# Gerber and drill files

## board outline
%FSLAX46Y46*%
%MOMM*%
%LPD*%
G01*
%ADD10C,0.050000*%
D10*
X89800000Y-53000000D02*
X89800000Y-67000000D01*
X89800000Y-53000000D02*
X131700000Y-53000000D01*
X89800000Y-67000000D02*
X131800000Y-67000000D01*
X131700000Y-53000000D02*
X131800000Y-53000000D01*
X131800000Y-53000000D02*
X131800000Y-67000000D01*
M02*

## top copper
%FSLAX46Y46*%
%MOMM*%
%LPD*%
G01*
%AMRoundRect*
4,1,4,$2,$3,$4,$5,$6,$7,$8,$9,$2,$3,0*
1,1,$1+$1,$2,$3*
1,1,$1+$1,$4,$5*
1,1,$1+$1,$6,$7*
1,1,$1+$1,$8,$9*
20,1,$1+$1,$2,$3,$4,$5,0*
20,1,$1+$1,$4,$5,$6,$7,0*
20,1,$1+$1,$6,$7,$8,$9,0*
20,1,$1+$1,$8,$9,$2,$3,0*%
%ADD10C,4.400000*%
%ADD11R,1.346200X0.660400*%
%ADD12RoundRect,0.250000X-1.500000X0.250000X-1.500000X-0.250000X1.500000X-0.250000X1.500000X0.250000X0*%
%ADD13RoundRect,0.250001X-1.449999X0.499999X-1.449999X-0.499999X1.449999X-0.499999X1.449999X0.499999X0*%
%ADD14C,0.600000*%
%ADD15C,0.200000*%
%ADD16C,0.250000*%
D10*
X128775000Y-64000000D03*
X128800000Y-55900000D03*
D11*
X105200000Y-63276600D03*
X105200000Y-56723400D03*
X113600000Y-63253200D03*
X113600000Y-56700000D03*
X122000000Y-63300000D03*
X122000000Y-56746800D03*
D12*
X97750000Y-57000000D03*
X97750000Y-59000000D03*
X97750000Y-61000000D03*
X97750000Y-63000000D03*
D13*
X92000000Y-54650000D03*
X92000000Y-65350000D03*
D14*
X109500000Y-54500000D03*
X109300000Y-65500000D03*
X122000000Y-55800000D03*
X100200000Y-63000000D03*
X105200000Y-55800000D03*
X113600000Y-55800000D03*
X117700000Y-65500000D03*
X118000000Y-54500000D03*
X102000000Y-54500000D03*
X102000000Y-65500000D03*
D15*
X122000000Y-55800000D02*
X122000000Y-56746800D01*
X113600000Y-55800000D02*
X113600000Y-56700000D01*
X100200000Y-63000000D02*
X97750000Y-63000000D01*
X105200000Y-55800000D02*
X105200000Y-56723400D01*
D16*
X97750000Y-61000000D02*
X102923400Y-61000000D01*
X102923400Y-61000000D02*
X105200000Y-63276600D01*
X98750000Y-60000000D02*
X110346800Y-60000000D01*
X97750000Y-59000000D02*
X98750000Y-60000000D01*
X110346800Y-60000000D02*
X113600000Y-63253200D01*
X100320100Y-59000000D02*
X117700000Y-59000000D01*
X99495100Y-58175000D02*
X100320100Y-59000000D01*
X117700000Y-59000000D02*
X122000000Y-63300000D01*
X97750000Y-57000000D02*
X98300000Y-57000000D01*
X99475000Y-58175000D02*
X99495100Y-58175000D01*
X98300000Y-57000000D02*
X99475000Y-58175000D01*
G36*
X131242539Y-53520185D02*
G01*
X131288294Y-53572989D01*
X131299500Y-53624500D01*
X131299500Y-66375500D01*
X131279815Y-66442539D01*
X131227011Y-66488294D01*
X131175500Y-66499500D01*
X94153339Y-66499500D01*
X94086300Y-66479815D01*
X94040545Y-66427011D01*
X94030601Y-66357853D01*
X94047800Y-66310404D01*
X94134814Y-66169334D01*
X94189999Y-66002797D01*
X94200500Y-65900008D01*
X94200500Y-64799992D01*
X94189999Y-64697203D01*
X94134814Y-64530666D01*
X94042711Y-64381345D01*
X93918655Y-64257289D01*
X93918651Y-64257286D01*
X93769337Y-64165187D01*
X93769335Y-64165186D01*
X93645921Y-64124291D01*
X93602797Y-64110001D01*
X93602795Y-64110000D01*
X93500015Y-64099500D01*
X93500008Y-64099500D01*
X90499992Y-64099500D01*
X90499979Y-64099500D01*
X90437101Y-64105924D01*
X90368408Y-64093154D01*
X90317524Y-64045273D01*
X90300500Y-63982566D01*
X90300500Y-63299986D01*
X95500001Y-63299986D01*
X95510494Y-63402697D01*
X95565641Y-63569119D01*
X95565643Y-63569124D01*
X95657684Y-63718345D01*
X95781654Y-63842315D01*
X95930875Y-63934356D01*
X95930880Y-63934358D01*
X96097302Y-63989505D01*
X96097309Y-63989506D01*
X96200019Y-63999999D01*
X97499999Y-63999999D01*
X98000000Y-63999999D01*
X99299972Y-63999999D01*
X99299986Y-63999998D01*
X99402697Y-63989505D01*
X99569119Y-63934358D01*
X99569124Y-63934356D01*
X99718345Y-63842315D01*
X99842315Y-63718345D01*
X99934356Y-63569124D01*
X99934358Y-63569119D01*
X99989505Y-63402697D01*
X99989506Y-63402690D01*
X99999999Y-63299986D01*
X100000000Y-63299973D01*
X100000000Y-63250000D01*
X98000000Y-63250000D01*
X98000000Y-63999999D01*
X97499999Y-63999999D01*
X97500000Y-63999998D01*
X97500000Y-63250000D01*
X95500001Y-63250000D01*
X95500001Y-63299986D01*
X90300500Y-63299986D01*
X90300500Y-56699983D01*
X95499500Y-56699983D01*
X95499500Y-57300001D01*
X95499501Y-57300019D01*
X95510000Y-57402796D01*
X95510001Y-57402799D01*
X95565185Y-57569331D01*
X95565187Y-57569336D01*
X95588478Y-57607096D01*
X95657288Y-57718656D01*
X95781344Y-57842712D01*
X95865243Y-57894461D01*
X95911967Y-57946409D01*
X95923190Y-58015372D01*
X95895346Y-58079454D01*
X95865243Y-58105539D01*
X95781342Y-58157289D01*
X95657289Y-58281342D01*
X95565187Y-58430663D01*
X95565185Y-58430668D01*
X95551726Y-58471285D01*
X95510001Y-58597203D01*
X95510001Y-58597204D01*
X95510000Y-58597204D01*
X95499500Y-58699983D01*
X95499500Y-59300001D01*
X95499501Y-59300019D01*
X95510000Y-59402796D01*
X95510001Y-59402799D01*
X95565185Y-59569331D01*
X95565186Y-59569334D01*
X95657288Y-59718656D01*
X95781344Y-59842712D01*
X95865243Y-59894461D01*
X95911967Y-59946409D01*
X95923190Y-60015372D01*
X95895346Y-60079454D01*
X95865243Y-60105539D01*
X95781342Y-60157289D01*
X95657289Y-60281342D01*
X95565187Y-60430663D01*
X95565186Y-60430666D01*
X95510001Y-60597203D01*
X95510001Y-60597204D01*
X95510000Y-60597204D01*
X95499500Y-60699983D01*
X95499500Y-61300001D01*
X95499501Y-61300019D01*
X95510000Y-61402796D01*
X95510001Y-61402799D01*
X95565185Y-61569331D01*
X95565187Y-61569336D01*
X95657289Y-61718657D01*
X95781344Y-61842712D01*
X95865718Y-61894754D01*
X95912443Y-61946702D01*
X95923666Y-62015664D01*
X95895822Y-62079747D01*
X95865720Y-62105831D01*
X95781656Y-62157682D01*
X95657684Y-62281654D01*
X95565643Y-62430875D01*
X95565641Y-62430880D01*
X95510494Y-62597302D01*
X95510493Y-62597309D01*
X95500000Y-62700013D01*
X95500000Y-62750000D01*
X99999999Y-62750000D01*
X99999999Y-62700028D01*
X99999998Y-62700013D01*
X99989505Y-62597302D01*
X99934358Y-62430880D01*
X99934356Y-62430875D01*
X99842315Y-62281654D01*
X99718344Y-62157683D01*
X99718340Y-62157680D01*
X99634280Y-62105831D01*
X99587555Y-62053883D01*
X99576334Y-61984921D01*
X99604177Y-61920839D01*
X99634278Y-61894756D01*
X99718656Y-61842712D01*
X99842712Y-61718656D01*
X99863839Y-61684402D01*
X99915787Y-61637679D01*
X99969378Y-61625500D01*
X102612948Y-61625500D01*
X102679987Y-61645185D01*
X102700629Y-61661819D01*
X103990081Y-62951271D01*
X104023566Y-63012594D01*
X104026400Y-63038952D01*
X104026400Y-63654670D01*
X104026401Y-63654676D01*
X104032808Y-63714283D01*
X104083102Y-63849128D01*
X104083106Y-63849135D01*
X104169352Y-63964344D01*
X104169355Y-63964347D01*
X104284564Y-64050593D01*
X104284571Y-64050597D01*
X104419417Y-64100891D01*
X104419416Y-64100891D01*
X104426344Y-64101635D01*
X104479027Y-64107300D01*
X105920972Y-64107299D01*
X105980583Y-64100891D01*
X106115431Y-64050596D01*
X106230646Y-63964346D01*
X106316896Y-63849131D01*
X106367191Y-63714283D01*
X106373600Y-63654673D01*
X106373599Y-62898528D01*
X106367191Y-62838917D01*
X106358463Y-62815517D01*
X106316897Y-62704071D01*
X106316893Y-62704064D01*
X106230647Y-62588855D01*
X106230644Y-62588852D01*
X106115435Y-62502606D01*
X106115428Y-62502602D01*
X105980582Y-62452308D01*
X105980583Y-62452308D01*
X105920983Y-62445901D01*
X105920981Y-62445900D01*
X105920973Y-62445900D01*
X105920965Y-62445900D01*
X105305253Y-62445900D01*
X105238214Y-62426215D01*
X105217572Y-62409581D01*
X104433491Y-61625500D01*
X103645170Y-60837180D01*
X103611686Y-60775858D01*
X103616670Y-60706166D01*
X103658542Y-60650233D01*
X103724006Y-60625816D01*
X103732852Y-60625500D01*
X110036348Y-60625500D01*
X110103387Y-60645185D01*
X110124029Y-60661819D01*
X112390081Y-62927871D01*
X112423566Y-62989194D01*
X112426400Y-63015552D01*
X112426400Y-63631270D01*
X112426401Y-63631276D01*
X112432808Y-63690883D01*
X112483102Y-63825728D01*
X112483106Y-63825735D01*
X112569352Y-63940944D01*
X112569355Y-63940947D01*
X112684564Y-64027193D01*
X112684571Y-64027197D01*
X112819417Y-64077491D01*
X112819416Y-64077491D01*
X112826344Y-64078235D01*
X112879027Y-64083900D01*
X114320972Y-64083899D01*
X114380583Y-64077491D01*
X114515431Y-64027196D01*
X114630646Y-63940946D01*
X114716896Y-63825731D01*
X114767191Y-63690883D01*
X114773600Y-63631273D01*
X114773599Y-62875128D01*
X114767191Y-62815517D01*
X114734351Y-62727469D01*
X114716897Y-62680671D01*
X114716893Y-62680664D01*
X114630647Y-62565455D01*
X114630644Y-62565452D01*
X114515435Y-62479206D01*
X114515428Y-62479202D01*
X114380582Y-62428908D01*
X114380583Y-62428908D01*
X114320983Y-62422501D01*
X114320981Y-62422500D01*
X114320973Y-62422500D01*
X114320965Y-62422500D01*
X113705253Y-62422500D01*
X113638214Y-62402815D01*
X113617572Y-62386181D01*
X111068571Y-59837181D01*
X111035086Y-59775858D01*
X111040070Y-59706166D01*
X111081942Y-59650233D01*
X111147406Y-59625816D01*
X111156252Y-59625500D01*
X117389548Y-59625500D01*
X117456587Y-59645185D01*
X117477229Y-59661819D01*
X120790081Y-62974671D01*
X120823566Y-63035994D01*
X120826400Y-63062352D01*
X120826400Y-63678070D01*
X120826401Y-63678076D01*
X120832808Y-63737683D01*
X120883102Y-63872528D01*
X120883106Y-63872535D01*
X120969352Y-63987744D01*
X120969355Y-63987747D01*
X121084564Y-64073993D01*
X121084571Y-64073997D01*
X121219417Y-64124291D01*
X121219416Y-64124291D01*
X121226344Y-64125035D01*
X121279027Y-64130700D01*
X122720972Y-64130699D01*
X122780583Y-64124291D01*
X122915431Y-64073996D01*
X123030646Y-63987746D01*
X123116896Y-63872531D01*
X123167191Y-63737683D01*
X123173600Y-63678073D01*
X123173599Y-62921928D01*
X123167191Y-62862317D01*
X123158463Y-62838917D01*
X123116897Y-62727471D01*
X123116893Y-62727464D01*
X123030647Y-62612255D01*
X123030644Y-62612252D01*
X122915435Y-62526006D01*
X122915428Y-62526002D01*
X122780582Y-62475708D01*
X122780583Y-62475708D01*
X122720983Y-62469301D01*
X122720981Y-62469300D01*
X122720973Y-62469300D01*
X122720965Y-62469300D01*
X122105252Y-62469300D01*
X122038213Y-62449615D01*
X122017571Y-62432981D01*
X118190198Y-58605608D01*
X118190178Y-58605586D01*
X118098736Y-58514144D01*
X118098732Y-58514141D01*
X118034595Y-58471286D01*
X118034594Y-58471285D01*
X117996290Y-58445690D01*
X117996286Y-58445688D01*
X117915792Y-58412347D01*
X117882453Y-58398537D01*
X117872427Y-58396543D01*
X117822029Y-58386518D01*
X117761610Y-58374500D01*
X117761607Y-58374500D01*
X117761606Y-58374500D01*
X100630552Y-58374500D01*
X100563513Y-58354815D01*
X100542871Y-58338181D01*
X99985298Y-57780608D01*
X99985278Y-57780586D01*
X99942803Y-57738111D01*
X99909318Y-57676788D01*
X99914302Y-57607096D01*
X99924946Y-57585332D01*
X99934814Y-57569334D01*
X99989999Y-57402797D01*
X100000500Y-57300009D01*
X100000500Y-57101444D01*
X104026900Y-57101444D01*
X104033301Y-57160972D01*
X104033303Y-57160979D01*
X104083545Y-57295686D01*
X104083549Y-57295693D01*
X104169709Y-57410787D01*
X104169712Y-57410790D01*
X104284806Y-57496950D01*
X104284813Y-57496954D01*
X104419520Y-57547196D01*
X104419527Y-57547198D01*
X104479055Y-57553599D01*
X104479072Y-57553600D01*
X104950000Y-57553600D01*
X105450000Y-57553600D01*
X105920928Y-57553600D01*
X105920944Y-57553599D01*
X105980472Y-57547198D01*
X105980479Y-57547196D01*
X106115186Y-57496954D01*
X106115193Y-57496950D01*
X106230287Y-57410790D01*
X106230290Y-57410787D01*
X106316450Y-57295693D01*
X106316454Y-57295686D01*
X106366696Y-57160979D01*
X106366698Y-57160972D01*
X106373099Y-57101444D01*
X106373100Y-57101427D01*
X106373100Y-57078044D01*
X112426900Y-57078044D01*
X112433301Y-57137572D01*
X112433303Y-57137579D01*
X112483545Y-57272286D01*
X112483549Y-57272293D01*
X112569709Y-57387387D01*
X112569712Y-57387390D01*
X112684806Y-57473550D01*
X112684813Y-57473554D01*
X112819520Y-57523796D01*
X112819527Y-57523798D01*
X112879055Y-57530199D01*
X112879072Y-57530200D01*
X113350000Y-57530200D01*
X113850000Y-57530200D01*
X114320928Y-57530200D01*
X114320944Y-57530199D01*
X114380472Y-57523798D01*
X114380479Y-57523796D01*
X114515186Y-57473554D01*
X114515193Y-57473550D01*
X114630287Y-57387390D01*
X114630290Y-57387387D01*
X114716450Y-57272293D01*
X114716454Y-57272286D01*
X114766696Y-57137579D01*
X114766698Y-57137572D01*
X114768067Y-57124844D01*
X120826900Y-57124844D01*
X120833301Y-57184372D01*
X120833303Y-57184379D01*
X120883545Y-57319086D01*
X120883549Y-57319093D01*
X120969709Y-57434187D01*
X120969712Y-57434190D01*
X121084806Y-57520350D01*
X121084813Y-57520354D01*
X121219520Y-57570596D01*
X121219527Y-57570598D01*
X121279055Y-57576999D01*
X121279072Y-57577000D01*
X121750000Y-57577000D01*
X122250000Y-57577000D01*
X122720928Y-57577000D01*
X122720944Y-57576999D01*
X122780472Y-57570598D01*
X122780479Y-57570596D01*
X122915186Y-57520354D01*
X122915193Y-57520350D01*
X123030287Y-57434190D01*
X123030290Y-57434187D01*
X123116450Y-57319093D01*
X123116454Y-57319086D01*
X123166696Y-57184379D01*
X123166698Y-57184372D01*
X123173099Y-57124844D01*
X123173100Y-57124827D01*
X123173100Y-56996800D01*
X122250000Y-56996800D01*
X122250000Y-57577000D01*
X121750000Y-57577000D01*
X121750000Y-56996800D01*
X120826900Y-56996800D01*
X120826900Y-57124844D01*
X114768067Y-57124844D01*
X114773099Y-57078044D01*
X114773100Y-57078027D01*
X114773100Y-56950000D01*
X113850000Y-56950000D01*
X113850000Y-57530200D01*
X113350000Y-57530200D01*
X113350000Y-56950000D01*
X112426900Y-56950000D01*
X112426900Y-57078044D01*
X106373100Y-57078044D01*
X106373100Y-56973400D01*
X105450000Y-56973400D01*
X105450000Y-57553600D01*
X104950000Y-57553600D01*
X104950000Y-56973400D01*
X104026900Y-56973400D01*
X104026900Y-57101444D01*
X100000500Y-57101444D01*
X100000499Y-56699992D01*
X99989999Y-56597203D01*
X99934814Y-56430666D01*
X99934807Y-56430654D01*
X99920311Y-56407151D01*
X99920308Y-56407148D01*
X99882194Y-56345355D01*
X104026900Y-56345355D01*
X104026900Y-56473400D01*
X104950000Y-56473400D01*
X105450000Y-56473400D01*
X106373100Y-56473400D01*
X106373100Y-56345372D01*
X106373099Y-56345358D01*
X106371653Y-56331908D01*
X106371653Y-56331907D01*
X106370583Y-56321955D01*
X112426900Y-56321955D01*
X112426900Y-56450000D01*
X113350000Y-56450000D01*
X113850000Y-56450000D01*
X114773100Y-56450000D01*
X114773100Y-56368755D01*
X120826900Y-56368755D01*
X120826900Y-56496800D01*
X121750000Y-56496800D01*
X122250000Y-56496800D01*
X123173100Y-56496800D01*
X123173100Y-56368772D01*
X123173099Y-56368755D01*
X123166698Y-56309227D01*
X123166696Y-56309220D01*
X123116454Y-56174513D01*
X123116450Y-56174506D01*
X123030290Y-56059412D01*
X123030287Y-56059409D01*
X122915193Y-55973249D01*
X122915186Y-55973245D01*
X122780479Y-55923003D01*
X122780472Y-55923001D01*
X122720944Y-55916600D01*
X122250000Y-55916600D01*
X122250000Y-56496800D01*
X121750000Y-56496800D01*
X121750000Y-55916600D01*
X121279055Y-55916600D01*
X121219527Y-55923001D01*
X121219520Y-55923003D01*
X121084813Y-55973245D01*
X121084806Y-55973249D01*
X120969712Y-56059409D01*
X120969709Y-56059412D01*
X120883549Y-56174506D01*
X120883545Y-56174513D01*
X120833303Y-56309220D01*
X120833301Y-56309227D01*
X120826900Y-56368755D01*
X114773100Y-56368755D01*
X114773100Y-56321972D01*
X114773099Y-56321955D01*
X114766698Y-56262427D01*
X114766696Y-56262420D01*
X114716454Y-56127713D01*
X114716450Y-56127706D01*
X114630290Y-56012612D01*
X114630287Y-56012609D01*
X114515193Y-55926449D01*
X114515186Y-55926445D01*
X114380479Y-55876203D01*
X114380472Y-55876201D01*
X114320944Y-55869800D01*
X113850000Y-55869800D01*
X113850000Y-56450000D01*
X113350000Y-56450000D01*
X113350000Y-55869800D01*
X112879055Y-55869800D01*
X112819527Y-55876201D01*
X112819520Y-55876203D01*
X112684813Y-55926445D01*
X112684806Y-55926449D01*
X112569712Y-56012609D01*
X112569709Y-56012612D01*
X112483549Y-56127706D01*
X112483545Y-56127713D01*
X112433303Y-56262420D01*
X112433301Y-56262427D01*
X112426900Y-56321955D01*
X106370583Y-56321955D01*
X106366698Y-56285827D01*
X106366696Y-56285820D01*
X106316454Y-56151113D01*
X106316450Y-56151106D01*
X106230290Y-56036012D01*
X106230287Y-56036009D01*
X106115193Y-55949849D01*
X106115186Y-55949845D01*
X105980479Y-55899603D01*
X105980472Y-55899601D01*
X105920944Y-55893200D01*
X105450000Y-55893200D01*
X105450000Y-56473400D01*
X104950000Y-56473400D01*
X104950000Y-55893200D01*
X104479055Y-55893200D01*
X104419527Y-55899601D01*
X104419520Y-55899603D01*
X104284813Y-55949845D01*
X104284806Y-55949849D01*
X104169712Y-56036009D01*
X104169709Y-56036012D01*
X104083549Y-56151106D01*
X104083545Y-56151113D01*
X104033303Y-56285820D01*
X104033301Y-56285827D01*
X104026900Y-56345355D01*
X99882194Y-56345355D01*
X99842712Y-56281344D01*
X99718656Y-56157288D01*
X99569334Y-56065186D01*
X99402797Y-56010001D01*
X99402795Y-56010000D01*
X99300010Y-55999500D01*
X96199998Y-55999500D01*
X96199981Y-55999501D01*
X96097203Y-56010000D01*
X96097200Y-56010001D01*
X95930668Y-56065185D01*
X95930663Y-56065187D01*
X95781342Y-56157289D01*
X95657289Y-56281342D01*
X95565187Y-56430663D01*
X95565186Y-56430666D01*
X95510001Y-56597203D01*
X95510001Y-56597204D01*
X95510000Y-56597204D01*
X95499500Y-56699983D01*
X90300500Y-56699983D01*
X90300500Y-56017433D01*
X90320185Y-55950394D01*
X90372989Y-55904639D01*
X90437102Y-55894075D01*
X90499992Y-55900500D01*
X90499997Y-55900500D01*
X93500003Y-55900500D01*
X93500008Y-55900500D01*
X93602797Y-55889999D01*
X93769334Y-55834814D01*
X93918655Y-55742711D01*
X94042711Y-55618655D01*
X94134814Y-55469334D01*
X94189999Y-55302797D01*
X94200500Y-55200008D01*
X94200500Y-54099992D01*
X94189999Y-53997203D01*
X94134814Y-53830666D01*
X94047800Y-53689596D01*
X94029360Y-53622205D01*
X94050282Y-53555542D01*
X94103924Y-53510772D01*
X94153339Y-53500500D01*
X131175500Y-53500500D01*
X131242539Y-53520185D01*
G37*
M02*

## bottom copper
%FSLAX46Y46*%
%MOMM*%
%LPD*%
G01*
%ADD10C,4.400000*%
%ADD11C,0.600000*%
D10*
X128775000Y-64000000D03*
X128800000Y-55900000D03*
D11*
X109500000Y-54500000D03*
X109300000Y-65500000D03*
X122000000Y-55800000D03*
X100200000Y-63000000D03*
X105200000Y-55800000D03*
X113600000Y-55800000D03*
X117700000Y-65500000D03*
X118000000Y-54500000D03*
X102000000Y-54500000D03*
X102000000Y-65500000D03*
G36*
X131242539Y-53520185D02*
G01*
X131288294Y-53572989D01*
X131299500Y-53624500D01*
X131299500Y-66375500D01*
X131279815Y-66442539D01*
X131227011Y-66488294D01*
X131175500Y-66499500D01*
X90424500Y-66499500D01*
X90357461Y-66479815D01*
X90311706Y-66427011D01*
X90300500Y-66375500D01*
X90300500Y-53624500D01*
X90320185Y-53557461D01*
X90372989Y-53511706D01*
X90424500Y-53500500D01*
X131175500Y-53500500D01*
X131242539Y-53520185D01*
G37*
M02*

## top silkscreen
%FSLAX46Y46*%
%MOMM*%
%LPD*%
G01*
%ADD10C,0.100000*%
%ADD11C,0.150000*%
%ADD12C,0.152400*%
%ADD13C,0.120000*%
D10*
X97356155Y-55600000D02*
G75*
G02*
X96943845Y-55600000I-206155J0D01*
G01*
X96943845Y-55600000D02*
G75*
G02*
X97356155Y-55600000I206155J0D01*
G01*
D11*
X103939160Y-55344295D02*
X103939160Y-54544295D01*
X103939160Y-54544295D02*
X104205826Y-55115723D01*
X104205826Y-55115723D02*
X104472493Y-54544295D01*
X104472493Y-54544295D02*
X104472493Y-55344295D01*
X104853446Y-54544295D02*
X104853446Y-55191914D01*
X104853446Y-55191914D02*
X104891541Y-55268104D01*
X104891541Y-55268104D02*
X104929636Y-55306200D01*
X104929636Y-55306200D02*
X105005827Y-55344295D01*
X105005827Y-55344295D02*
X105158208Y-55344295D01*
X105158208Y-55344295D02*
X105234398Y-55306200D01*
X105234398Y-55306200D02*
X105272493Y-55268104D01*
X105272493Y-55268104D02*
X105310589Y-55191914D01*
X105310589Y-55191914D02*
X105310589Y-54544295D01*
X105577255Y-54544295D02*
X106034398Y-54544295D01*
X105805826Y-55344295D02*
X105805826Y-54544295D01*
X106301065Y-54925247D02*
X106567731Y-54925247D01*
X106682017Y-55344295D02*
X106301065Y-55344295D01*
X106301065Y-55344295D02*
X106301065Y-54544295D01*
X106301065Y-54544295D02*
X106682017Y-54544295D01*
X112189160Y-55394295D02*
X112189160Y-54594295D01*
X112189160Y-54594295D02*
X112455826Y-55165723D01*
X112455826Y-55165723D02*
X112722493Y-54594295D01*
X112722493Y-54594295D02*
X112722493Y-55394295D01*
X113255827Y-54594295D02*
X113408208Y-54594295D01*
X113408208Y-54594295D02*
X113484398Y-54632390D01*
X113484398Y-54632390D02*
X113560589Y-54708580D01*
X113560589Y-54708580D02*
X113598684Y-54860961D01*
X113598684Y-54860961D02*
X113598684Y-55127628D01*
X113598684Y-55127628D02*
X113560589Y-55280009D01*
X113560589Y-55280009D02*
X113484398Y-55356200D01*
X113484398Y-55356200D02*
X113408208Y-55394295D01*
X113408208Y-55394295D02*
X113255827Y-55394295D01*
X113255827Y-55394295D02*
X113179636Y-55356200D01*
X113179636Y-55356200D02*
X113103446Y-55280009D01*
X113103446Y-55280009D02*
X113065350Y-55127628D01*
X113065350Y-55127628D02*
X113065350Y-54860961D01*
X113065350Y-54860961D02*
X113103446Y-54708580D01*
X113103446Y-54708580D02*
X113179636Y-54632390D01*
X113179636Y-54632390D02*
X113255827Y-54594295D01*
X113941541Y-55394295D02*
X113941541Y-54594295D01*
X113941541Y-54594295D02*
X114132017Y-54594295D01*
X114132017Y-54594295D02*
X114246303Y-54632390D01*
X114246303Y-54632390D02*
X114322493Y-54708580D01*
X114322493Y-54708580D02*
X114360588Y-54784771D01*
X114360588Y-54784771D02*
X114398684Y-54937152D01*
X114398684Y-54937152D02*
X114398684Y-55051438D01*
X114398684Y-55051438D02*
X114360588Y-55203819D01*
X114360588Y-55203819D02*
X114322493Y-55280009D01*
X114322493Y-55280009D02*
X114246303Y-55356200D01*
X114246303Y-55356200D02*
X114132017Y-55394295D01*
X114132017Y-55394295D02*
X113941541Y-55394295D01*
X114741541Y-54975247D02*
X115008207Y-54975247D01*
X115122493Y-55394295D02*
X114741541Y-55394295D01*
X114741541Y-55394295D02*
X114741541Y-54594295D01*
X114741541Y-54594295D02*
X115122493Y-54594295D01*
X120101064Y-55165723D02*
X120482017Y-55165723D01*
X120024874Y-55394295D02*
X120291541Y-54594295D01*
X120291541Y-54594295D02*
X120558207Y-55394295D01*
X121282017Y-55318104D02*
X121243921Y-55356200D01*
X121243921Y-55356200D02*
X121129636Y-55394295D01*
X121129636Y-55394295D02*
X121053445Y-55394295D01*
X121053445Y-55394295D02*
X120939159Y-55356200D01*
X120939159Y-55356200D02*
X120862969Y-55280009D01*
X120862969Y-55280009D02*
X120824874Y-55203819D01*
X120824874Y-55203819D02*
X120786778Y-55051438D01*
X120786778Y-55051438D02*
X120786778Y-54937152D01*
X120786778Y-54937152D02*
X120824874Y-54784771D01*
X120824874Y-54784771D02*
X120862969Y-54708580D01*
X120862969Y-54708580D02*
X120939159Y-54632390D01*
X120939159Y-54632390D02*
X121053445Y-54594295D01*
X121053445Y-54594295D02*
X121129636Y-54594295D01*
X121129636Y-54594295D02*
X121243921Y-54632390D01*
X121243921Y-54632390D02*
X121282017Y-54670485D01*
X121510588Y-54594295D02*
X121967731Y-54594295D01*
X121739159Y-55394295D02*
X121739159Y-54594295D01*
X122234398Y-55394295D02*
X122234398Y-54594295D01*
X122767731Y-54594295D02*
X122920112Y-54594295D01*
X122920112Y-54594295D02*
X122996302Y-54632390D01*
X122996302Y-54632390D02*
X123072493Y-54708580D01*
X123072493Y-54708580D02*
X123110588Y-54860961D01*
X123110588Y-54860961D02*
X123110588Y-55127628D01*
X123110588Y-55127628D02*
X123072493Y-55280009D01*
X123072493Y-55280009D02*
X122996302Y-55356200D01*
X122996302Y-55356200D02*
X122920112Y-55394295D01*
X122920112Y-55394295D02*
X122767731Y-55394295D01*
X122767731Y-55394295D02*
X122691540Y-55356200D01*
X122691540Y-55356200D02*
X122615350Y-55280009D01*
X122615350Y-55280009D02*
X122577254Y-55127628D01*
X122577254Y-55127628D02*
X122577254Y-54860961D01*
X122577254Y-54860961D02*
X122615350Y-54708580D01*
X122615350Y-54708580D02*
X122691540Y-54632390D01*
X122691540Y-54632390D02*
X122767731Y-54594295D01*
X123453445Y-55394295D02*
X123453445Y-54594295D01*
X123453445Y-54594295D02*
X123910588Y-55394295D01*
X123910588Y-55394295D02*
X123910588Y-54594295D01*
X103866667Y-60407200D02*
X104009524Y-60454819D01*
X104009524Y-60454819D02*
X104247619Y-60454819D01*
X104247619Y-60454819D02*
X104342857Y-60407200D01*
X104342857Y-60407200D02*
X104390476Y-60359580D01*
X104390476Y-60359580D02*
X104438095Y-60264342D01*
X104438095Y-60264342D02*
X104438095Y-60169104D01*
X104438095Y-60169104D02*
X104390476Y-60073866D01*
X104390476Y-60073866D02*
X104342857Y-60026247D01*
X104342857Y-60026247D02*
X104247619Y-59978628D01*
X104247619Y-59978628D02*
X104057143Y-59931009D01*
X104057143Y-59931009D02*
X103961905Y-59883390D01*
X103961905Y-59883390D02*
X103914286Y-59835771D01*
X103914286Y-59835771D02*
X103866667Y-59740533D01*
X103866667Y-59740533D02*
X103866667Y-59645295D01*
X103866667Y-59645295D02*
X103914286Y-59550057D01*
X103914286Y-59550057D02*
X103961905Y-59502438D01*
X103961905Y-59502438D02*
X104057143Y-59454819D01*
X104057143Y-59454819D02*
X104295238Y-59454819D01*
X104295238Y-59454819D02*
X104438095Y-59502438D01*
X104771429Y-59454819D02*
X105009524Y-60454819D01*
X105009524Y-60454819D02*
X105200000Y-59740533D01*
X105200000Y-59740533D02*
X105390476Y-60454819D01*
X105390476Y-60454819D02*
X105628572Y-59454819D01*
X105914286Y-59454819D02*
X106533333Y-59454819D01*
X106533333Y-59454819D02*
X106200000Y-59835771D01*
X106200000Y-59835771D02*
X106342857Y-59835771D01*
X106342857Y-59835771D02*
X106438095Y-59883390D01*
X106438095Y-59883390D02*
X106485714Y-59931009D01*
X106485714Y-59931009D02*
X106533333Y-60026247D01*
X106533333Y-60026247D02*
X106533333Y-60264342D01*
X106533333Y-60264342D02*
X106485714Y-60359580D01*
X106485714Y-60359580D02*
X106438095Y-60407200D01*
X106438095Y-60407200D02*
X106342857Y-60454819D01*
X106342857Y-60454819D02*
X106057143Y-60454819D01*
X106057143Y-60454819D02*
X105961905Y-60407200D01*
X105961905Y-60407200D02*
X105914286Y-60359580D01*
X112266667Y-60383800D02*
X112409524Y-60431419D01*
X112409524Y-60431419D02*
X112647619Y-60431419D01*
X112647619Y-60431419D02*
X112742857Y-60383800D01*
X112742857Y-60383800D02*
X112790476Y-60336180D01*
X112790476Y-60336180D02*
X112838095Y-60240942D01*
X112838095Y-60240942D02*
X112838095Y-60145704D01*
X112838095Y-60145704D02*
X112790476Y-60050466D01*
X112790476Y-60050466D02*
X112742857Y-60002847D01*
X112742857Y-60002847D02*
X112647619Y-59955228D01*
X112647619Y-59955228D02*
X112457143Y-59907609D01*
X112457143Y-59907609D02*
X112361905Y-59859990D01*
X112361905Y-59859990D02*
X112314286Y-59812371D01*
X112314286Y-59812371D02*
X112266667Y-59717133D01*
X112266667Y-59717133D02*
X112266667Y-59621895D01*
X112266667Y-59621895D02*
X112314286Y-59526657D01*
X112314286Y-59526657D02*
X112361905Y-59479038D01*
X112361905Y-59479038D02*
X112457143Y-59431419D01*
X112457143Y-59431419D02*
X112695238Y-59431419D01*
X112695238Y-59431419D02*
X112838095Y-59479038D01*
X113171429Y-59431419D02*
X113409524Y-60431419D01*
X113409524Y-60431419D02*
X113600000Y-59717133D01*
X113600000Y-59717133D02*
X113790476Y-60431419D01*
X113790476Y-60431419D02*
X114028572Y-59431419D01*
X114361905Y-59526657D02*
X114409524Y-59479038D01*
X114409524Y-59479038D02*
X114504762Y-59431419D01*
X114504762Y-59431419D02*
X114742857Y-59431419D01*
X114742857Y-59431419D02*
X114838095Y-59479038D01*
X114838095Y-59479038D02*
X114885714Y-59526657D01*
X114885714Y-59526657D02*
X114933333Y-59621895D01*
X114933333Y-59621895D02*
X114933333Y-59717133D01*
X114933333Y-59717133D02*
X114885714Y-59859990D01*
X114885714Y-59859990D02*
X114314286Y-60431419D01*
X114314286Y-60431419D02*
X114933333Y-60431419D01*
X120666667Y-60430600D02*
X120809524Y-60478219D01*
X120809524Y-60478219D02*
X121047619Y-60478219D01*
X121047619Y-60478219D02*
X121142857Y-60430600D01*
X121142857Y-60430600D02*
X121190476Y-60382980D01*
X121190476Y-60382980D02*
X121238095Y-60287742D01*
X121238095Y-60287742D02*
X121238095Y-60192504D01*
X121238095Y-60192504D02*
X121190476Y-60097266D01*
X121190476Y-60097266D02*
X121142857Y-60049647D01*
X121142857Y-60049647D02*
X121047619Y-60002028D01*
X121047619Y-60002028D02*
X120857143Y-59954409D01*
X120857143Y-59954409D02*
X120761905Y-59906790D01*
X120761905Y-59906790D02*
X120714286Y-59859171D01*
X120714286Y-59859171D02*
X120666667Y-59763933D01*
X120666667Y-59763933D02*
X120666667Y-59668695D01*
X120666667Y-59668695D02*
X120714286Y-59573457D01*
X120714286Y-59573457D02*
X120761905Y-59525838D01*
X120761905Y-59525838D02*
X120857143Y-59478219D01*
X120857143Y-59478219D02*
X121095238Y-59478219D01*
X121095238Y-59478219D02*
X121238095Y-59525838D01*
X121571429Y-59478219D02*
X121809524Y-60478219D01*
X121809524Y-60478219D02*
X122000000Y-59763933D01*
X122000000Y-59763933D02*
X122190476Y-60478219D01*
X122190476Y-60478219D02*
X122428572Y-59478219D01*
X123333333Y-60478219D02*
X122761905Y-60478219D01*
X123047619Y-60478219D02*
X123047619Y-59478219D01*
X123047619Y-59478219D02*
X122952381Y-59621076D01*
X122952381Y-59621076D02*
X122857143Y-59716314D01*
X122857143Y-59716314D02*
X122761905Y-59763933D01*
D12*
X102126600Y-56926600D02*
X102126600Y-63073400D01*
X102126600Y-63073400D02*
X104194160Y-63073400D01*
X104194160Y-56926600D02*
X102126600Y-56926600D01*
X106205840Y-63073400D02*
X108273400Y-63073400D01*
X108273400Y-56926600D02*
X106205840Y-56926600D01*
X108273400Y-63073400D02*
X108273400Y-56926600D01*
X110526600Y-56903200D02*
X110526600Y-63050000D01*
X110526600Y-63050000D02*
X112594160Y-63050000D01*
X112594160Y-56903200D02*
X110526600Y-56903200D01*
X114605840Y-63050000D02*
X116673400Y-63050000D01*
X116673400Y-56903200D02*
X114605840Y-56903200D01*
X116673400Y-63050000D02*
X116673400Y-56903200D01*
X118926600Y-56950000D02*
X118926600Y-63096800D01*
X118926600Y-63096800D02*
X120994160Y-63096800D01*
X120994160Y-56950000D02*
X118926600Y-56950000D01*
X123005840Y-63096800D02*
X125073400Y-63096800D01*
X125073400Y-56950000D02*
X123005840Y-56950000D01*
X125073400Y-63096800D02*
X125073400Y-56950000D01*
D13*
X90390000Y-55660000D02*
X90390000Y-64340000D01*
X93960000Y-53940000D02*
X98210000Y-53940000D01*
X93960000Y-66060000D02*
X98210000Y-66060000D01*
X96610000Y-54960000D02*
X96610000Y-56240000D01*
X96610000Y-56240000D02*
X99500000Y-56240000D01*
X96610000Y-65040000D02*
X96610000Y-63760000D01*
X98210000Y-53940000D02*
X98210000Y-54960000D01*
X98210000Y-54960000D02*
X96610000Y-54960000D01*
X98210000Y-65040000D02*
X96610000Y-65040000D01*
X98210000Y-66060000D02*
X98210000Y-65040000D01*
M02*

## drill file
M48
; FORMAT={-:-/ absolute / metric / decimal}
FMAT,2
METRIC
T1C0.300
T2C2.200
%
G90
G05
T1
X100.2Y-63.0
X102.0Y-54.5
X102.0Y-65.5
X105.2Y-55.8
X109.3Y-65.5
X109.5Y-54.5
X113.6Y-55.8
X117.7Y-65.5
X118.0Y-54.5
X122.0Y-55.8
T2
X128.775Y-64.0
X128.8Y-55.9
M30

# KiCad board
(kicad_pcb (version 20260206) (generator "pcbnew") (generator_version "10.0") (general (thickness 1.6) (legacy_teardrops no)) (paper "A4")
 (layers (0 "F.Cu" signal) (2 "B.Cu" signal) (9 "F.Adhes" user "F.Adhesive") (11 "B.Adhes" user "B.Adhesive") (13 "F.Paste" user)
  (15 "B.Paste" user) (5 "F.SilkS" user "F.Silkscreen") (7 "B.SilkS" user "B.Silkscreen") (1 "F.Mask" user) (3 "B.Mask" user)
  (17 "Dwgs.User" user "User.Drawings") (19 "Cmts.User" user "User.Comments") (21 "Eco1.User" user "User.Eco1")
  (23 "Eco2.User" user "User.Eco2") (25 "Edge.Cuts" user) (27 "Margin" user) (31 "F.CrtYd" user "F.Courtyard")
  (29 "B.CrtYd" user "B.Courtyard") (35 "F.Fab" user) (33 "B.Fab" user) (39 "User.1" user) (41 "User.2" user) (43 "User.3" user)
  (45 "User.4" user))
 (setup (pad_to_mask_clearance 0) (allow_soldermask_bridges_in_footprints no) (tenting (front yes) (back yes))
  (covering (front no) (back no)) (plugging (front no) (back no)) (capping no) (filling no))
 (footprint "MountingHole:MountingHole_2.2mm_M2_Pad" (layer "F.Cu") (at 128.775 64)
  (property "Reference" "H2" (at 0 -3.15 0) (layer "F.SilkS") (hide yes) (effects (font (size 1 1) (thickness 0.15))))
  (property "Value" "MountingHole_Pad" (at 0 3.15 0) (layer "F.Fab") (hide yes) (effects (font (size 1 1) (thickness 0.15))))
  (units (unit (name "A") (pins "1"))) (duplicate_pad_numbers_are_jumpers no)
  (pad "1" thru_hole circle (at 0 0) (size 4.4 4.4) (drill 2.2) (layers "*.Cu" "*.Mask") (remove_unused_layers no) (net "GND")
   (zone_connect 2)))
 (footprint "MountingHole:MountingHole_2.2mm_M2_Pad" (layer "F.Cu") (at 128.8 55.9)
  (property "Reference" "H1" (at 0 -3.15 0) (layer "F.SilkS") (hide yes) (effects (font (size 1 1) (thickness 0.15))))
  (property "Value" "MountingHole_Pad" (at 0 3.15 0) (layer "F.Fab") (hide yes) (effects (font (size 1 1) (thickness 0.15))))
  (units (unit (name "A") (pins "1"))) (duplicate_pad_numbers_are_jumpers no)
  (pad "1" thru_hole circle (at 0 0) (size 4.4 4.4) (drill 2.2) (layers "*.Cu" "*.Mask") (remove_unused_layers no) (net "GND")
   (zone_connect 2)))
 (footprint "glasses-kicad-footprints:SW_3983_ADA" (layer "F.Cu") (at 105.2 60 90)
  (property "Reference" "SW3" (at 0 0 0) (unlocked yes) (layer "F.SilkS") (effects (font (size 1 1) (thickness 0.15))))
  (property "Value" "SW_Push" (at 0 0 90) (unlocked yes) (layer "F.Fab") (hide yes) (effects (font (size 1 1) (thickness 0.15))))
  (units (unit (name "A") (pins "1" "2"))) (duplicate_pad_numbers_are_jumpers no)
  (fp_line (start 3.0734 -3.0734) (end -3.0734 -3.0734) (stroke (width 0.1524) (type solid)) (layer "F.SilkS"))
  (fp_line (start -3.0734 -3.0734) (end -3.0734 -1.00584) (stroke (width 0.1524) (type solid)) (layer "F.SilkS"))
  (fp_line (start 3.0734 -1.00584) (end 3.0734 -3.0734) (stroke (width 0.1524) (type solid)) (layer "F.SilkS"))
  (fp_line (start -3.0734 1.00584) (end -3.0734 3.0734) (stroke (width 0.1524) (type solid)) (layer "F.SilkS"))
  (fp_line (start 3.0734 3.0734) (end 3.0734 1.00584) (stroke (width 0.1524) (type solid)) (layer "F.SilkS"))
  (fp_line (start -3.0734 3.0734) (end 3.0734 3.0734) (stroke (width 0.1524) (type solid)) (layer "F.SilkS"))
  (pad "1" smd rect (at -3.2766 0 90) (size 0.6604 1.3462) (layers "F.Cu" "F.Mask" "F.Paste") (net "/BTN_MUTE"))
  (pad "2" smd rect (at 3.2766 0 90) (size 0.6604 1.3462) (layers "F.Cu" "F.Mask" "F.Paste") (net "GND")))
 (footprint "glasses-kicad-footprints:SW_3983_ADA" (layer "F.Cu") (at 113.6 59.9766 90)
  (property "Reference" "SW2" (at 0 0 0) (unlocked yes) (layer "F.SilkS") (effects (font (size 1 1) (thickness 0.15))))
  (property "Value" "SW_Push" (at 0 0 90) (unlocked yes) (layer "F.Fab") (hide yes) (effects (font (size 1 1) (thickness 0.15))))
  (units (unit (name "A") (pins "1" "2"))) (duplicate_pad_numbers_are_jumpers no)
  (fp_line (start 3.0734 -3.0734) (end -3.0734 -3.0734) (stroke (width 0.1524) (type solid)) (layer "F.SilkS"))
  (fp_line (start -3.0734 -3.0734) (end -3.0734 -1.00584) (stroke (width 0.1524) (type solid)) (layer "F.SilkS"))
  (fp_line (start 3.0734 -1.00584) (end 3.0734 -3.0734) (stroke (width 0.1524) (type solid)) (layer "F.SilkS"))
  (fp_line (start -3.0734 1.00584) (end -3.0734 3.0734) (stroke (width 0.1524) (type solid)) (layer "F.SilkS"))
  (fp_line (start 3.0734 3.0734) (end 3.0734 1.00584) (stroke (width 0.1524) (type solid)) (layer "F.SilkS"))
  (fp_line (start -3.0734 3.0734) (end 3.0734 3.0734) (stroke (width 0.1524) (type solid)) (layer "F.SilkS"))
  (pad "1" smd rect (at -3.2766 0 90) (size 0.6604 1.3462) (layers "F.Cu" "F.Mask" "F.Paste") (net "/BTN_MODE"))
  (pad "2" smd rect (at 3.2766 0 90) (size 0.6604 1.3462) (layers "F.Cu" "F.Mask" "F.Paste") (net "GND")))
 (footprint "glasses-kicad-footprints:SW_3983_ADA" (layer "F.Cu") (at 122 60.0234 90)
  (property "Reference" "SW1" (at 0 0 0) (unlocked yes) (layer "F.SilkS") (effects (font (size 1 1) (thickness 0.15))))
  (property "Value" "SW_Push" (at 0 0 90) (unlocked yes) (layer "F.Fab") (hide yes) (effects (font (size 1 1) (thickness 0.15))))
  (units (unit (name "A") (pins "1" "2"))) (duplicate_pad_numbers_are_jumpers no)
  (fp_line (start 3.0734 -3.0734) (end -3.0734 -3.0734) (stroke (width 0.1524) (type solid)) (layer "F.SilkS"))
  (fp_line (start -3.0734 -3.0734) (end -3.0734 -1.00584) (stroke (width 0.1524) (type solid)) (layer "F.SilkS"))
  (fp_line (start 3.0734 -1.00584) (end 3.0734 -3.0734) (stroke (width 0.1524) (type solid)) (layer "F.SilkS"))
  (fp_line (start -3.0734 1.00584) (end -3.0734 3.0734) (stroke (width 0.1524) (type solid)) (layer "F.SilkS"))
  (fp_line (start 3.0734 3.0734) (end 3.0734 1.00584) (stroke (width 0.1524) (type solid)) (layer "F.SilkS"))
  (fp_line (start -3.0734 3.0734) (end 3.0734 3.0734) (stroke (width 0.1524) (type solid)) (layer "F.SilkS"))
  (pad "1" smd rect (at -3.2766 0 90) (size 0.6604 1.3462) (layers "F.Cu" "F.Mask" "F.Paste") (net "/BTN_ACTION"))
  (pad "2" smd rect (at 3.2766 0 90) (size 0.6604 1.3462) (layers "F.Cu" "F.Mask" "F.Paste") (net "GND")))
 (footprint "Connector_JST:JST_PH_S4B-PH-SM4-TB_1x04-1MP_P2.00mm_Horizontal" (layer "F.Cu") (at 94.9 60 -90)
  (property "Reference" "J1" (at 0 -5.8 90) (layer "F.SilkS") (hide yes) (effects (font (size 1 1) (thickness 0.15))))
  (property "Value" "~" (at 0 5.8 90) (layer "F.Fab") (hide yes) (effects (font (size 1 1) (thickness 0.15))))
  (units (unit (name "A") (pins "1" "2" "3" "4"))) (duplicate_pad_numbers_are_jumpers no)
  (fp_line (start -4.34 4.51) (end 4.34 4.51) (stroke (width 0.12) (type solid)) (layer "F.SilkS"))
  (fp_line (start -6.06 0.94) (end -6.06 -3.31) (stroke (width 0.12) (type solid)) (layer "F.SilkS"))
  (fp_line (start 6.06 0.94) (end 6.06 -3.31) (stroke (width 0.12) (type solid)) (layer "F.SilkS"))
  (fp_line (start -5.04 -1.71) (end -3.76 -1.71) (stroke (width 0.12) (type solid)) (layer "F.SilkS"))
  (fp_line (start -3.76 -1.71) (end -3.76 -4.6) (stroke (width 0.12) (type solid)) (layer "F.SilkS"))
  (fp_line (start 5.04 -1.71) (end 3.76 -1.71) (stroke (width 0.12) (type solid)) (layer "F.SilkS"))
  (fp_line (start -6.06 -3.31) (end -5.04 -3.31) (stroke (width 0.12) (type solid)) (layer "F.SilkS"))
  (fp_line (start -5.04 -3.31) (end -5.04 -1.71) (stroke (width 0.12) (type solid)) (layer "F.SilkS"))
  (fp_line (start 5.04 -3.31) (end 5.04 -1.71) (stroke (width 0.12) (type solid)) (layer "F.SilkS"))
  (fp_line (start 6.06 -3.31) (end 5.04 -3.31) (stroke (width 0.12) (type solid)) (layer "F.SilkS"))
  (pad "1" smd roundrect (at -3 -2.85 270) (size 1 3.5) (layers "F.Cu" "F.Mask" "F.Paste") (roundrect_rratio 0.25) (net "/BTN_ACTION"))
  (pad "2" smd roundrect (at -1 -2.85 270) (size 1 3.5) (layers "F.Cu" "F.Mask" "F.Paste") (roundrect_rratio 0.25) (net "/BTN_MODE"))
  (pad "3" smd roundrect (at 1 -2.85 270) (size 1 3.5) (layers "F.Cu" "F.Mask" "F.Paste") (roundrect_rratio 0.25) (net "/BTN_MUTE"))
  (pad "4" smd roundrect (at 3 -2.85 270) (size 1 3.5) (layers "F.Cu" "F.Mask" "F.Paste") (roundrect_rratio 0.25) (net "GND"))
  (pad "MP" smd roundrect (at -5.35 2.9 270) (size 1.5 3.4) (layers "F.Cu" "F.Mask" "F.Paste") (roundrect_rratio 0.166667))
  (pad "MP" smd roundrect (at 5.35 2.9 270) (size 1.5 3.4) (layers "F.Cu" "F.Mask" "F.Paste") (roundrect_rratio 0.166667)))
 (gr_circle (center 97.15 55.6) (end 97.2 55.8) (stroke (width 0.1) (type default)) (fill no) (layer "F.SilkS"))
 (gr_line (start 89.8 53) (end 89.8 67) (stroke (width 0.05) (type default)) (layer "Edge.Cuts"))
 (gr_line (start 89.8 53) (end 131.7 53) (stroke (width 0.05) (type default)) (layer "Edge.Cuts"))
 (gr_line (start 89.8 67) (end 131.8 67) (stroke (width 0.05) (type default)) (layer "Edge.Cuts"))
 (gr_line (start 131.7 53) (end 131.8 53) (stroke (width 0.05) (type default)) (layer "Edge.Cuts"))
 (gr_line (start 131.8 53) (end 131.8 67) (stroke (width 0.05) (type default)) (layer "Edge.Cuts"))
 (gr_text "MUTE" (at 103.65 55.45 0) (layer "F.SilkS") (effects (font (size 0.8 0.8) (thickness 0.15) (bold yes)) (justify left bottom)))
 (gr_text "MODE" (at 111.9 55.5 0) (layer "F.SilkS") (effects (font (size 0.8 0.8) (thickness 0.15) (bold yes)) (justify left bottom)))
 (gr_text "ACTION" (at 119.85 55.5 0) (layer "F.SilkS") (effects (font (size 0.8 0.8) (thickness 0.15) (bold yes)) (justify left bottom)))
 (segment (start 122 55.8) (end 122 56.7468) (width 0.2) (layer "F.Cu") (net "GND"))
 (segment (start 113.6 55.8) (end 113.6 56.7) (width 0.2) (layer "F.Cu") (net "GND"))
 (segment (start 100.2 63) (end 97.75 63) (width 0.2) (layer "F.Cu") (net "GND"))
 (segment (start 105.2 55.8) (end 105.2 56.7234) (width 0.2) (layer "F.Cu") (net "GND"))
 (via (at 109.5 54.5) (size 0.6) (drill 0.3) (layers "F.Cu" "B.Cu") (free yes) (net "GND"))
 (via (at 109.3 65.5) (size 0.6) (drill 0.3) (layers "F.Cu" "B.Cu") (free yes) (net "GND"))
 (via (at 122 55.8) (size 0.6) (drill 0.3) (layers "F.Cu" "B.Cu") (free yes) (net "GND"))
 (via (at 100.2 63) (size 0.6) (drill 0.3) (layers "F.Cu" "B.Cu") (free yes) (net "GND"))
 (via (at 105.2 55.8) (size 0.6) (drill 0.3) (layers "F.Cu" "B.Cu") (free yes) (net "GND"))
 (via (at 113.6 55.8) (size 0.6) (drill 0.3) (layers "F.Cu" "B.Cu") (free yes) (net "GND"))
 (via (at 117.7 65.5) (size 0.6) (drill 0.3) (layers "F.Cu" "B.Cu") (free yes) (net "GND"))
 (via (at 118 54.5) (size 0.6) (drill 0.3) (layers "F.Cu" "B.Cu") (free yes) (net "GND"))
 (via (at 102 54.5) (size 0.6) (drill 0.3) (layers "F.Cu" "B.Cu") (free yes) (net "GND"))
 (via (at 102 65.5) (size 0.6) (drill 0.3) (layers "F.Cu" "B.Cu") (free yes) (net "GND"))
 (segment (start 97.75 61) (end 102.9234 61) (width 0.25) (layer "F.Cu") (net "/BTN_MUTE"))
 (segment (start 102.9234 61) (end 105.2 63.2766) (width 0.25) (layer "F.Cu") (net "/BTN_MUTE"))
 (segment (start 98.75 60) (end 110.3468 60) (width 0.25) (layer "F.Cu") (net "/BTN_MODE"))
 (segment (start 97.75 59) (end 98.75 60) (width 0.25) (layer "F.Cu") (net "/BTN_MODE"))
 (segment (start 110.3468 60) (end 113.6 63.2532) (width 0.25) (layer "F.Cu") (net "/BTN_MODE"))
 (segment (start 100.3201 59) (end 117.7 59) (width 0.25) (layer "F.Cu") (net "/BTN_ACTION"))
 (segment (start 99.4951 58.175) (end 100.3201 59) (width 0.25) (layer "F.Cu") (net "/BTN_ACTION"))
 (segment (start 117.7 59) (end 122 63.3) (width 0.25) (layer "F.Cu") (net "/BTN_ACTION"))
 (segment (start 97.75 57) (end 98.3 57) (width 0.25) (layer "F.Cu") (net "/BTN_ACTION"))
 (segment (start 99.475 58.175) (end 99.4951 58.175) (width 0.25) (layer "F.Cu") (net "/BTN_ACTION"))
 (segment (start 98.3 57) (end 99.475 58.175) (width 0.25) (layer "F.Cu") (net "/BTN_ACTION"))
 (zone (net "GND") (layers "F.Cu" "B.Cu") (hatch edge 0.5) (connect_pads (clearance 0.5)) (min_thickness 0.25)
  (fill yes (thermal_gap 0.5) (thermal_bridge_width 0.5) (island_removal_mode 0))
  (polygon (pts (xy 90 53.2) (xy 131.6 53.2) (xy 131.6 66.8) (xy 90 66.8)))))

